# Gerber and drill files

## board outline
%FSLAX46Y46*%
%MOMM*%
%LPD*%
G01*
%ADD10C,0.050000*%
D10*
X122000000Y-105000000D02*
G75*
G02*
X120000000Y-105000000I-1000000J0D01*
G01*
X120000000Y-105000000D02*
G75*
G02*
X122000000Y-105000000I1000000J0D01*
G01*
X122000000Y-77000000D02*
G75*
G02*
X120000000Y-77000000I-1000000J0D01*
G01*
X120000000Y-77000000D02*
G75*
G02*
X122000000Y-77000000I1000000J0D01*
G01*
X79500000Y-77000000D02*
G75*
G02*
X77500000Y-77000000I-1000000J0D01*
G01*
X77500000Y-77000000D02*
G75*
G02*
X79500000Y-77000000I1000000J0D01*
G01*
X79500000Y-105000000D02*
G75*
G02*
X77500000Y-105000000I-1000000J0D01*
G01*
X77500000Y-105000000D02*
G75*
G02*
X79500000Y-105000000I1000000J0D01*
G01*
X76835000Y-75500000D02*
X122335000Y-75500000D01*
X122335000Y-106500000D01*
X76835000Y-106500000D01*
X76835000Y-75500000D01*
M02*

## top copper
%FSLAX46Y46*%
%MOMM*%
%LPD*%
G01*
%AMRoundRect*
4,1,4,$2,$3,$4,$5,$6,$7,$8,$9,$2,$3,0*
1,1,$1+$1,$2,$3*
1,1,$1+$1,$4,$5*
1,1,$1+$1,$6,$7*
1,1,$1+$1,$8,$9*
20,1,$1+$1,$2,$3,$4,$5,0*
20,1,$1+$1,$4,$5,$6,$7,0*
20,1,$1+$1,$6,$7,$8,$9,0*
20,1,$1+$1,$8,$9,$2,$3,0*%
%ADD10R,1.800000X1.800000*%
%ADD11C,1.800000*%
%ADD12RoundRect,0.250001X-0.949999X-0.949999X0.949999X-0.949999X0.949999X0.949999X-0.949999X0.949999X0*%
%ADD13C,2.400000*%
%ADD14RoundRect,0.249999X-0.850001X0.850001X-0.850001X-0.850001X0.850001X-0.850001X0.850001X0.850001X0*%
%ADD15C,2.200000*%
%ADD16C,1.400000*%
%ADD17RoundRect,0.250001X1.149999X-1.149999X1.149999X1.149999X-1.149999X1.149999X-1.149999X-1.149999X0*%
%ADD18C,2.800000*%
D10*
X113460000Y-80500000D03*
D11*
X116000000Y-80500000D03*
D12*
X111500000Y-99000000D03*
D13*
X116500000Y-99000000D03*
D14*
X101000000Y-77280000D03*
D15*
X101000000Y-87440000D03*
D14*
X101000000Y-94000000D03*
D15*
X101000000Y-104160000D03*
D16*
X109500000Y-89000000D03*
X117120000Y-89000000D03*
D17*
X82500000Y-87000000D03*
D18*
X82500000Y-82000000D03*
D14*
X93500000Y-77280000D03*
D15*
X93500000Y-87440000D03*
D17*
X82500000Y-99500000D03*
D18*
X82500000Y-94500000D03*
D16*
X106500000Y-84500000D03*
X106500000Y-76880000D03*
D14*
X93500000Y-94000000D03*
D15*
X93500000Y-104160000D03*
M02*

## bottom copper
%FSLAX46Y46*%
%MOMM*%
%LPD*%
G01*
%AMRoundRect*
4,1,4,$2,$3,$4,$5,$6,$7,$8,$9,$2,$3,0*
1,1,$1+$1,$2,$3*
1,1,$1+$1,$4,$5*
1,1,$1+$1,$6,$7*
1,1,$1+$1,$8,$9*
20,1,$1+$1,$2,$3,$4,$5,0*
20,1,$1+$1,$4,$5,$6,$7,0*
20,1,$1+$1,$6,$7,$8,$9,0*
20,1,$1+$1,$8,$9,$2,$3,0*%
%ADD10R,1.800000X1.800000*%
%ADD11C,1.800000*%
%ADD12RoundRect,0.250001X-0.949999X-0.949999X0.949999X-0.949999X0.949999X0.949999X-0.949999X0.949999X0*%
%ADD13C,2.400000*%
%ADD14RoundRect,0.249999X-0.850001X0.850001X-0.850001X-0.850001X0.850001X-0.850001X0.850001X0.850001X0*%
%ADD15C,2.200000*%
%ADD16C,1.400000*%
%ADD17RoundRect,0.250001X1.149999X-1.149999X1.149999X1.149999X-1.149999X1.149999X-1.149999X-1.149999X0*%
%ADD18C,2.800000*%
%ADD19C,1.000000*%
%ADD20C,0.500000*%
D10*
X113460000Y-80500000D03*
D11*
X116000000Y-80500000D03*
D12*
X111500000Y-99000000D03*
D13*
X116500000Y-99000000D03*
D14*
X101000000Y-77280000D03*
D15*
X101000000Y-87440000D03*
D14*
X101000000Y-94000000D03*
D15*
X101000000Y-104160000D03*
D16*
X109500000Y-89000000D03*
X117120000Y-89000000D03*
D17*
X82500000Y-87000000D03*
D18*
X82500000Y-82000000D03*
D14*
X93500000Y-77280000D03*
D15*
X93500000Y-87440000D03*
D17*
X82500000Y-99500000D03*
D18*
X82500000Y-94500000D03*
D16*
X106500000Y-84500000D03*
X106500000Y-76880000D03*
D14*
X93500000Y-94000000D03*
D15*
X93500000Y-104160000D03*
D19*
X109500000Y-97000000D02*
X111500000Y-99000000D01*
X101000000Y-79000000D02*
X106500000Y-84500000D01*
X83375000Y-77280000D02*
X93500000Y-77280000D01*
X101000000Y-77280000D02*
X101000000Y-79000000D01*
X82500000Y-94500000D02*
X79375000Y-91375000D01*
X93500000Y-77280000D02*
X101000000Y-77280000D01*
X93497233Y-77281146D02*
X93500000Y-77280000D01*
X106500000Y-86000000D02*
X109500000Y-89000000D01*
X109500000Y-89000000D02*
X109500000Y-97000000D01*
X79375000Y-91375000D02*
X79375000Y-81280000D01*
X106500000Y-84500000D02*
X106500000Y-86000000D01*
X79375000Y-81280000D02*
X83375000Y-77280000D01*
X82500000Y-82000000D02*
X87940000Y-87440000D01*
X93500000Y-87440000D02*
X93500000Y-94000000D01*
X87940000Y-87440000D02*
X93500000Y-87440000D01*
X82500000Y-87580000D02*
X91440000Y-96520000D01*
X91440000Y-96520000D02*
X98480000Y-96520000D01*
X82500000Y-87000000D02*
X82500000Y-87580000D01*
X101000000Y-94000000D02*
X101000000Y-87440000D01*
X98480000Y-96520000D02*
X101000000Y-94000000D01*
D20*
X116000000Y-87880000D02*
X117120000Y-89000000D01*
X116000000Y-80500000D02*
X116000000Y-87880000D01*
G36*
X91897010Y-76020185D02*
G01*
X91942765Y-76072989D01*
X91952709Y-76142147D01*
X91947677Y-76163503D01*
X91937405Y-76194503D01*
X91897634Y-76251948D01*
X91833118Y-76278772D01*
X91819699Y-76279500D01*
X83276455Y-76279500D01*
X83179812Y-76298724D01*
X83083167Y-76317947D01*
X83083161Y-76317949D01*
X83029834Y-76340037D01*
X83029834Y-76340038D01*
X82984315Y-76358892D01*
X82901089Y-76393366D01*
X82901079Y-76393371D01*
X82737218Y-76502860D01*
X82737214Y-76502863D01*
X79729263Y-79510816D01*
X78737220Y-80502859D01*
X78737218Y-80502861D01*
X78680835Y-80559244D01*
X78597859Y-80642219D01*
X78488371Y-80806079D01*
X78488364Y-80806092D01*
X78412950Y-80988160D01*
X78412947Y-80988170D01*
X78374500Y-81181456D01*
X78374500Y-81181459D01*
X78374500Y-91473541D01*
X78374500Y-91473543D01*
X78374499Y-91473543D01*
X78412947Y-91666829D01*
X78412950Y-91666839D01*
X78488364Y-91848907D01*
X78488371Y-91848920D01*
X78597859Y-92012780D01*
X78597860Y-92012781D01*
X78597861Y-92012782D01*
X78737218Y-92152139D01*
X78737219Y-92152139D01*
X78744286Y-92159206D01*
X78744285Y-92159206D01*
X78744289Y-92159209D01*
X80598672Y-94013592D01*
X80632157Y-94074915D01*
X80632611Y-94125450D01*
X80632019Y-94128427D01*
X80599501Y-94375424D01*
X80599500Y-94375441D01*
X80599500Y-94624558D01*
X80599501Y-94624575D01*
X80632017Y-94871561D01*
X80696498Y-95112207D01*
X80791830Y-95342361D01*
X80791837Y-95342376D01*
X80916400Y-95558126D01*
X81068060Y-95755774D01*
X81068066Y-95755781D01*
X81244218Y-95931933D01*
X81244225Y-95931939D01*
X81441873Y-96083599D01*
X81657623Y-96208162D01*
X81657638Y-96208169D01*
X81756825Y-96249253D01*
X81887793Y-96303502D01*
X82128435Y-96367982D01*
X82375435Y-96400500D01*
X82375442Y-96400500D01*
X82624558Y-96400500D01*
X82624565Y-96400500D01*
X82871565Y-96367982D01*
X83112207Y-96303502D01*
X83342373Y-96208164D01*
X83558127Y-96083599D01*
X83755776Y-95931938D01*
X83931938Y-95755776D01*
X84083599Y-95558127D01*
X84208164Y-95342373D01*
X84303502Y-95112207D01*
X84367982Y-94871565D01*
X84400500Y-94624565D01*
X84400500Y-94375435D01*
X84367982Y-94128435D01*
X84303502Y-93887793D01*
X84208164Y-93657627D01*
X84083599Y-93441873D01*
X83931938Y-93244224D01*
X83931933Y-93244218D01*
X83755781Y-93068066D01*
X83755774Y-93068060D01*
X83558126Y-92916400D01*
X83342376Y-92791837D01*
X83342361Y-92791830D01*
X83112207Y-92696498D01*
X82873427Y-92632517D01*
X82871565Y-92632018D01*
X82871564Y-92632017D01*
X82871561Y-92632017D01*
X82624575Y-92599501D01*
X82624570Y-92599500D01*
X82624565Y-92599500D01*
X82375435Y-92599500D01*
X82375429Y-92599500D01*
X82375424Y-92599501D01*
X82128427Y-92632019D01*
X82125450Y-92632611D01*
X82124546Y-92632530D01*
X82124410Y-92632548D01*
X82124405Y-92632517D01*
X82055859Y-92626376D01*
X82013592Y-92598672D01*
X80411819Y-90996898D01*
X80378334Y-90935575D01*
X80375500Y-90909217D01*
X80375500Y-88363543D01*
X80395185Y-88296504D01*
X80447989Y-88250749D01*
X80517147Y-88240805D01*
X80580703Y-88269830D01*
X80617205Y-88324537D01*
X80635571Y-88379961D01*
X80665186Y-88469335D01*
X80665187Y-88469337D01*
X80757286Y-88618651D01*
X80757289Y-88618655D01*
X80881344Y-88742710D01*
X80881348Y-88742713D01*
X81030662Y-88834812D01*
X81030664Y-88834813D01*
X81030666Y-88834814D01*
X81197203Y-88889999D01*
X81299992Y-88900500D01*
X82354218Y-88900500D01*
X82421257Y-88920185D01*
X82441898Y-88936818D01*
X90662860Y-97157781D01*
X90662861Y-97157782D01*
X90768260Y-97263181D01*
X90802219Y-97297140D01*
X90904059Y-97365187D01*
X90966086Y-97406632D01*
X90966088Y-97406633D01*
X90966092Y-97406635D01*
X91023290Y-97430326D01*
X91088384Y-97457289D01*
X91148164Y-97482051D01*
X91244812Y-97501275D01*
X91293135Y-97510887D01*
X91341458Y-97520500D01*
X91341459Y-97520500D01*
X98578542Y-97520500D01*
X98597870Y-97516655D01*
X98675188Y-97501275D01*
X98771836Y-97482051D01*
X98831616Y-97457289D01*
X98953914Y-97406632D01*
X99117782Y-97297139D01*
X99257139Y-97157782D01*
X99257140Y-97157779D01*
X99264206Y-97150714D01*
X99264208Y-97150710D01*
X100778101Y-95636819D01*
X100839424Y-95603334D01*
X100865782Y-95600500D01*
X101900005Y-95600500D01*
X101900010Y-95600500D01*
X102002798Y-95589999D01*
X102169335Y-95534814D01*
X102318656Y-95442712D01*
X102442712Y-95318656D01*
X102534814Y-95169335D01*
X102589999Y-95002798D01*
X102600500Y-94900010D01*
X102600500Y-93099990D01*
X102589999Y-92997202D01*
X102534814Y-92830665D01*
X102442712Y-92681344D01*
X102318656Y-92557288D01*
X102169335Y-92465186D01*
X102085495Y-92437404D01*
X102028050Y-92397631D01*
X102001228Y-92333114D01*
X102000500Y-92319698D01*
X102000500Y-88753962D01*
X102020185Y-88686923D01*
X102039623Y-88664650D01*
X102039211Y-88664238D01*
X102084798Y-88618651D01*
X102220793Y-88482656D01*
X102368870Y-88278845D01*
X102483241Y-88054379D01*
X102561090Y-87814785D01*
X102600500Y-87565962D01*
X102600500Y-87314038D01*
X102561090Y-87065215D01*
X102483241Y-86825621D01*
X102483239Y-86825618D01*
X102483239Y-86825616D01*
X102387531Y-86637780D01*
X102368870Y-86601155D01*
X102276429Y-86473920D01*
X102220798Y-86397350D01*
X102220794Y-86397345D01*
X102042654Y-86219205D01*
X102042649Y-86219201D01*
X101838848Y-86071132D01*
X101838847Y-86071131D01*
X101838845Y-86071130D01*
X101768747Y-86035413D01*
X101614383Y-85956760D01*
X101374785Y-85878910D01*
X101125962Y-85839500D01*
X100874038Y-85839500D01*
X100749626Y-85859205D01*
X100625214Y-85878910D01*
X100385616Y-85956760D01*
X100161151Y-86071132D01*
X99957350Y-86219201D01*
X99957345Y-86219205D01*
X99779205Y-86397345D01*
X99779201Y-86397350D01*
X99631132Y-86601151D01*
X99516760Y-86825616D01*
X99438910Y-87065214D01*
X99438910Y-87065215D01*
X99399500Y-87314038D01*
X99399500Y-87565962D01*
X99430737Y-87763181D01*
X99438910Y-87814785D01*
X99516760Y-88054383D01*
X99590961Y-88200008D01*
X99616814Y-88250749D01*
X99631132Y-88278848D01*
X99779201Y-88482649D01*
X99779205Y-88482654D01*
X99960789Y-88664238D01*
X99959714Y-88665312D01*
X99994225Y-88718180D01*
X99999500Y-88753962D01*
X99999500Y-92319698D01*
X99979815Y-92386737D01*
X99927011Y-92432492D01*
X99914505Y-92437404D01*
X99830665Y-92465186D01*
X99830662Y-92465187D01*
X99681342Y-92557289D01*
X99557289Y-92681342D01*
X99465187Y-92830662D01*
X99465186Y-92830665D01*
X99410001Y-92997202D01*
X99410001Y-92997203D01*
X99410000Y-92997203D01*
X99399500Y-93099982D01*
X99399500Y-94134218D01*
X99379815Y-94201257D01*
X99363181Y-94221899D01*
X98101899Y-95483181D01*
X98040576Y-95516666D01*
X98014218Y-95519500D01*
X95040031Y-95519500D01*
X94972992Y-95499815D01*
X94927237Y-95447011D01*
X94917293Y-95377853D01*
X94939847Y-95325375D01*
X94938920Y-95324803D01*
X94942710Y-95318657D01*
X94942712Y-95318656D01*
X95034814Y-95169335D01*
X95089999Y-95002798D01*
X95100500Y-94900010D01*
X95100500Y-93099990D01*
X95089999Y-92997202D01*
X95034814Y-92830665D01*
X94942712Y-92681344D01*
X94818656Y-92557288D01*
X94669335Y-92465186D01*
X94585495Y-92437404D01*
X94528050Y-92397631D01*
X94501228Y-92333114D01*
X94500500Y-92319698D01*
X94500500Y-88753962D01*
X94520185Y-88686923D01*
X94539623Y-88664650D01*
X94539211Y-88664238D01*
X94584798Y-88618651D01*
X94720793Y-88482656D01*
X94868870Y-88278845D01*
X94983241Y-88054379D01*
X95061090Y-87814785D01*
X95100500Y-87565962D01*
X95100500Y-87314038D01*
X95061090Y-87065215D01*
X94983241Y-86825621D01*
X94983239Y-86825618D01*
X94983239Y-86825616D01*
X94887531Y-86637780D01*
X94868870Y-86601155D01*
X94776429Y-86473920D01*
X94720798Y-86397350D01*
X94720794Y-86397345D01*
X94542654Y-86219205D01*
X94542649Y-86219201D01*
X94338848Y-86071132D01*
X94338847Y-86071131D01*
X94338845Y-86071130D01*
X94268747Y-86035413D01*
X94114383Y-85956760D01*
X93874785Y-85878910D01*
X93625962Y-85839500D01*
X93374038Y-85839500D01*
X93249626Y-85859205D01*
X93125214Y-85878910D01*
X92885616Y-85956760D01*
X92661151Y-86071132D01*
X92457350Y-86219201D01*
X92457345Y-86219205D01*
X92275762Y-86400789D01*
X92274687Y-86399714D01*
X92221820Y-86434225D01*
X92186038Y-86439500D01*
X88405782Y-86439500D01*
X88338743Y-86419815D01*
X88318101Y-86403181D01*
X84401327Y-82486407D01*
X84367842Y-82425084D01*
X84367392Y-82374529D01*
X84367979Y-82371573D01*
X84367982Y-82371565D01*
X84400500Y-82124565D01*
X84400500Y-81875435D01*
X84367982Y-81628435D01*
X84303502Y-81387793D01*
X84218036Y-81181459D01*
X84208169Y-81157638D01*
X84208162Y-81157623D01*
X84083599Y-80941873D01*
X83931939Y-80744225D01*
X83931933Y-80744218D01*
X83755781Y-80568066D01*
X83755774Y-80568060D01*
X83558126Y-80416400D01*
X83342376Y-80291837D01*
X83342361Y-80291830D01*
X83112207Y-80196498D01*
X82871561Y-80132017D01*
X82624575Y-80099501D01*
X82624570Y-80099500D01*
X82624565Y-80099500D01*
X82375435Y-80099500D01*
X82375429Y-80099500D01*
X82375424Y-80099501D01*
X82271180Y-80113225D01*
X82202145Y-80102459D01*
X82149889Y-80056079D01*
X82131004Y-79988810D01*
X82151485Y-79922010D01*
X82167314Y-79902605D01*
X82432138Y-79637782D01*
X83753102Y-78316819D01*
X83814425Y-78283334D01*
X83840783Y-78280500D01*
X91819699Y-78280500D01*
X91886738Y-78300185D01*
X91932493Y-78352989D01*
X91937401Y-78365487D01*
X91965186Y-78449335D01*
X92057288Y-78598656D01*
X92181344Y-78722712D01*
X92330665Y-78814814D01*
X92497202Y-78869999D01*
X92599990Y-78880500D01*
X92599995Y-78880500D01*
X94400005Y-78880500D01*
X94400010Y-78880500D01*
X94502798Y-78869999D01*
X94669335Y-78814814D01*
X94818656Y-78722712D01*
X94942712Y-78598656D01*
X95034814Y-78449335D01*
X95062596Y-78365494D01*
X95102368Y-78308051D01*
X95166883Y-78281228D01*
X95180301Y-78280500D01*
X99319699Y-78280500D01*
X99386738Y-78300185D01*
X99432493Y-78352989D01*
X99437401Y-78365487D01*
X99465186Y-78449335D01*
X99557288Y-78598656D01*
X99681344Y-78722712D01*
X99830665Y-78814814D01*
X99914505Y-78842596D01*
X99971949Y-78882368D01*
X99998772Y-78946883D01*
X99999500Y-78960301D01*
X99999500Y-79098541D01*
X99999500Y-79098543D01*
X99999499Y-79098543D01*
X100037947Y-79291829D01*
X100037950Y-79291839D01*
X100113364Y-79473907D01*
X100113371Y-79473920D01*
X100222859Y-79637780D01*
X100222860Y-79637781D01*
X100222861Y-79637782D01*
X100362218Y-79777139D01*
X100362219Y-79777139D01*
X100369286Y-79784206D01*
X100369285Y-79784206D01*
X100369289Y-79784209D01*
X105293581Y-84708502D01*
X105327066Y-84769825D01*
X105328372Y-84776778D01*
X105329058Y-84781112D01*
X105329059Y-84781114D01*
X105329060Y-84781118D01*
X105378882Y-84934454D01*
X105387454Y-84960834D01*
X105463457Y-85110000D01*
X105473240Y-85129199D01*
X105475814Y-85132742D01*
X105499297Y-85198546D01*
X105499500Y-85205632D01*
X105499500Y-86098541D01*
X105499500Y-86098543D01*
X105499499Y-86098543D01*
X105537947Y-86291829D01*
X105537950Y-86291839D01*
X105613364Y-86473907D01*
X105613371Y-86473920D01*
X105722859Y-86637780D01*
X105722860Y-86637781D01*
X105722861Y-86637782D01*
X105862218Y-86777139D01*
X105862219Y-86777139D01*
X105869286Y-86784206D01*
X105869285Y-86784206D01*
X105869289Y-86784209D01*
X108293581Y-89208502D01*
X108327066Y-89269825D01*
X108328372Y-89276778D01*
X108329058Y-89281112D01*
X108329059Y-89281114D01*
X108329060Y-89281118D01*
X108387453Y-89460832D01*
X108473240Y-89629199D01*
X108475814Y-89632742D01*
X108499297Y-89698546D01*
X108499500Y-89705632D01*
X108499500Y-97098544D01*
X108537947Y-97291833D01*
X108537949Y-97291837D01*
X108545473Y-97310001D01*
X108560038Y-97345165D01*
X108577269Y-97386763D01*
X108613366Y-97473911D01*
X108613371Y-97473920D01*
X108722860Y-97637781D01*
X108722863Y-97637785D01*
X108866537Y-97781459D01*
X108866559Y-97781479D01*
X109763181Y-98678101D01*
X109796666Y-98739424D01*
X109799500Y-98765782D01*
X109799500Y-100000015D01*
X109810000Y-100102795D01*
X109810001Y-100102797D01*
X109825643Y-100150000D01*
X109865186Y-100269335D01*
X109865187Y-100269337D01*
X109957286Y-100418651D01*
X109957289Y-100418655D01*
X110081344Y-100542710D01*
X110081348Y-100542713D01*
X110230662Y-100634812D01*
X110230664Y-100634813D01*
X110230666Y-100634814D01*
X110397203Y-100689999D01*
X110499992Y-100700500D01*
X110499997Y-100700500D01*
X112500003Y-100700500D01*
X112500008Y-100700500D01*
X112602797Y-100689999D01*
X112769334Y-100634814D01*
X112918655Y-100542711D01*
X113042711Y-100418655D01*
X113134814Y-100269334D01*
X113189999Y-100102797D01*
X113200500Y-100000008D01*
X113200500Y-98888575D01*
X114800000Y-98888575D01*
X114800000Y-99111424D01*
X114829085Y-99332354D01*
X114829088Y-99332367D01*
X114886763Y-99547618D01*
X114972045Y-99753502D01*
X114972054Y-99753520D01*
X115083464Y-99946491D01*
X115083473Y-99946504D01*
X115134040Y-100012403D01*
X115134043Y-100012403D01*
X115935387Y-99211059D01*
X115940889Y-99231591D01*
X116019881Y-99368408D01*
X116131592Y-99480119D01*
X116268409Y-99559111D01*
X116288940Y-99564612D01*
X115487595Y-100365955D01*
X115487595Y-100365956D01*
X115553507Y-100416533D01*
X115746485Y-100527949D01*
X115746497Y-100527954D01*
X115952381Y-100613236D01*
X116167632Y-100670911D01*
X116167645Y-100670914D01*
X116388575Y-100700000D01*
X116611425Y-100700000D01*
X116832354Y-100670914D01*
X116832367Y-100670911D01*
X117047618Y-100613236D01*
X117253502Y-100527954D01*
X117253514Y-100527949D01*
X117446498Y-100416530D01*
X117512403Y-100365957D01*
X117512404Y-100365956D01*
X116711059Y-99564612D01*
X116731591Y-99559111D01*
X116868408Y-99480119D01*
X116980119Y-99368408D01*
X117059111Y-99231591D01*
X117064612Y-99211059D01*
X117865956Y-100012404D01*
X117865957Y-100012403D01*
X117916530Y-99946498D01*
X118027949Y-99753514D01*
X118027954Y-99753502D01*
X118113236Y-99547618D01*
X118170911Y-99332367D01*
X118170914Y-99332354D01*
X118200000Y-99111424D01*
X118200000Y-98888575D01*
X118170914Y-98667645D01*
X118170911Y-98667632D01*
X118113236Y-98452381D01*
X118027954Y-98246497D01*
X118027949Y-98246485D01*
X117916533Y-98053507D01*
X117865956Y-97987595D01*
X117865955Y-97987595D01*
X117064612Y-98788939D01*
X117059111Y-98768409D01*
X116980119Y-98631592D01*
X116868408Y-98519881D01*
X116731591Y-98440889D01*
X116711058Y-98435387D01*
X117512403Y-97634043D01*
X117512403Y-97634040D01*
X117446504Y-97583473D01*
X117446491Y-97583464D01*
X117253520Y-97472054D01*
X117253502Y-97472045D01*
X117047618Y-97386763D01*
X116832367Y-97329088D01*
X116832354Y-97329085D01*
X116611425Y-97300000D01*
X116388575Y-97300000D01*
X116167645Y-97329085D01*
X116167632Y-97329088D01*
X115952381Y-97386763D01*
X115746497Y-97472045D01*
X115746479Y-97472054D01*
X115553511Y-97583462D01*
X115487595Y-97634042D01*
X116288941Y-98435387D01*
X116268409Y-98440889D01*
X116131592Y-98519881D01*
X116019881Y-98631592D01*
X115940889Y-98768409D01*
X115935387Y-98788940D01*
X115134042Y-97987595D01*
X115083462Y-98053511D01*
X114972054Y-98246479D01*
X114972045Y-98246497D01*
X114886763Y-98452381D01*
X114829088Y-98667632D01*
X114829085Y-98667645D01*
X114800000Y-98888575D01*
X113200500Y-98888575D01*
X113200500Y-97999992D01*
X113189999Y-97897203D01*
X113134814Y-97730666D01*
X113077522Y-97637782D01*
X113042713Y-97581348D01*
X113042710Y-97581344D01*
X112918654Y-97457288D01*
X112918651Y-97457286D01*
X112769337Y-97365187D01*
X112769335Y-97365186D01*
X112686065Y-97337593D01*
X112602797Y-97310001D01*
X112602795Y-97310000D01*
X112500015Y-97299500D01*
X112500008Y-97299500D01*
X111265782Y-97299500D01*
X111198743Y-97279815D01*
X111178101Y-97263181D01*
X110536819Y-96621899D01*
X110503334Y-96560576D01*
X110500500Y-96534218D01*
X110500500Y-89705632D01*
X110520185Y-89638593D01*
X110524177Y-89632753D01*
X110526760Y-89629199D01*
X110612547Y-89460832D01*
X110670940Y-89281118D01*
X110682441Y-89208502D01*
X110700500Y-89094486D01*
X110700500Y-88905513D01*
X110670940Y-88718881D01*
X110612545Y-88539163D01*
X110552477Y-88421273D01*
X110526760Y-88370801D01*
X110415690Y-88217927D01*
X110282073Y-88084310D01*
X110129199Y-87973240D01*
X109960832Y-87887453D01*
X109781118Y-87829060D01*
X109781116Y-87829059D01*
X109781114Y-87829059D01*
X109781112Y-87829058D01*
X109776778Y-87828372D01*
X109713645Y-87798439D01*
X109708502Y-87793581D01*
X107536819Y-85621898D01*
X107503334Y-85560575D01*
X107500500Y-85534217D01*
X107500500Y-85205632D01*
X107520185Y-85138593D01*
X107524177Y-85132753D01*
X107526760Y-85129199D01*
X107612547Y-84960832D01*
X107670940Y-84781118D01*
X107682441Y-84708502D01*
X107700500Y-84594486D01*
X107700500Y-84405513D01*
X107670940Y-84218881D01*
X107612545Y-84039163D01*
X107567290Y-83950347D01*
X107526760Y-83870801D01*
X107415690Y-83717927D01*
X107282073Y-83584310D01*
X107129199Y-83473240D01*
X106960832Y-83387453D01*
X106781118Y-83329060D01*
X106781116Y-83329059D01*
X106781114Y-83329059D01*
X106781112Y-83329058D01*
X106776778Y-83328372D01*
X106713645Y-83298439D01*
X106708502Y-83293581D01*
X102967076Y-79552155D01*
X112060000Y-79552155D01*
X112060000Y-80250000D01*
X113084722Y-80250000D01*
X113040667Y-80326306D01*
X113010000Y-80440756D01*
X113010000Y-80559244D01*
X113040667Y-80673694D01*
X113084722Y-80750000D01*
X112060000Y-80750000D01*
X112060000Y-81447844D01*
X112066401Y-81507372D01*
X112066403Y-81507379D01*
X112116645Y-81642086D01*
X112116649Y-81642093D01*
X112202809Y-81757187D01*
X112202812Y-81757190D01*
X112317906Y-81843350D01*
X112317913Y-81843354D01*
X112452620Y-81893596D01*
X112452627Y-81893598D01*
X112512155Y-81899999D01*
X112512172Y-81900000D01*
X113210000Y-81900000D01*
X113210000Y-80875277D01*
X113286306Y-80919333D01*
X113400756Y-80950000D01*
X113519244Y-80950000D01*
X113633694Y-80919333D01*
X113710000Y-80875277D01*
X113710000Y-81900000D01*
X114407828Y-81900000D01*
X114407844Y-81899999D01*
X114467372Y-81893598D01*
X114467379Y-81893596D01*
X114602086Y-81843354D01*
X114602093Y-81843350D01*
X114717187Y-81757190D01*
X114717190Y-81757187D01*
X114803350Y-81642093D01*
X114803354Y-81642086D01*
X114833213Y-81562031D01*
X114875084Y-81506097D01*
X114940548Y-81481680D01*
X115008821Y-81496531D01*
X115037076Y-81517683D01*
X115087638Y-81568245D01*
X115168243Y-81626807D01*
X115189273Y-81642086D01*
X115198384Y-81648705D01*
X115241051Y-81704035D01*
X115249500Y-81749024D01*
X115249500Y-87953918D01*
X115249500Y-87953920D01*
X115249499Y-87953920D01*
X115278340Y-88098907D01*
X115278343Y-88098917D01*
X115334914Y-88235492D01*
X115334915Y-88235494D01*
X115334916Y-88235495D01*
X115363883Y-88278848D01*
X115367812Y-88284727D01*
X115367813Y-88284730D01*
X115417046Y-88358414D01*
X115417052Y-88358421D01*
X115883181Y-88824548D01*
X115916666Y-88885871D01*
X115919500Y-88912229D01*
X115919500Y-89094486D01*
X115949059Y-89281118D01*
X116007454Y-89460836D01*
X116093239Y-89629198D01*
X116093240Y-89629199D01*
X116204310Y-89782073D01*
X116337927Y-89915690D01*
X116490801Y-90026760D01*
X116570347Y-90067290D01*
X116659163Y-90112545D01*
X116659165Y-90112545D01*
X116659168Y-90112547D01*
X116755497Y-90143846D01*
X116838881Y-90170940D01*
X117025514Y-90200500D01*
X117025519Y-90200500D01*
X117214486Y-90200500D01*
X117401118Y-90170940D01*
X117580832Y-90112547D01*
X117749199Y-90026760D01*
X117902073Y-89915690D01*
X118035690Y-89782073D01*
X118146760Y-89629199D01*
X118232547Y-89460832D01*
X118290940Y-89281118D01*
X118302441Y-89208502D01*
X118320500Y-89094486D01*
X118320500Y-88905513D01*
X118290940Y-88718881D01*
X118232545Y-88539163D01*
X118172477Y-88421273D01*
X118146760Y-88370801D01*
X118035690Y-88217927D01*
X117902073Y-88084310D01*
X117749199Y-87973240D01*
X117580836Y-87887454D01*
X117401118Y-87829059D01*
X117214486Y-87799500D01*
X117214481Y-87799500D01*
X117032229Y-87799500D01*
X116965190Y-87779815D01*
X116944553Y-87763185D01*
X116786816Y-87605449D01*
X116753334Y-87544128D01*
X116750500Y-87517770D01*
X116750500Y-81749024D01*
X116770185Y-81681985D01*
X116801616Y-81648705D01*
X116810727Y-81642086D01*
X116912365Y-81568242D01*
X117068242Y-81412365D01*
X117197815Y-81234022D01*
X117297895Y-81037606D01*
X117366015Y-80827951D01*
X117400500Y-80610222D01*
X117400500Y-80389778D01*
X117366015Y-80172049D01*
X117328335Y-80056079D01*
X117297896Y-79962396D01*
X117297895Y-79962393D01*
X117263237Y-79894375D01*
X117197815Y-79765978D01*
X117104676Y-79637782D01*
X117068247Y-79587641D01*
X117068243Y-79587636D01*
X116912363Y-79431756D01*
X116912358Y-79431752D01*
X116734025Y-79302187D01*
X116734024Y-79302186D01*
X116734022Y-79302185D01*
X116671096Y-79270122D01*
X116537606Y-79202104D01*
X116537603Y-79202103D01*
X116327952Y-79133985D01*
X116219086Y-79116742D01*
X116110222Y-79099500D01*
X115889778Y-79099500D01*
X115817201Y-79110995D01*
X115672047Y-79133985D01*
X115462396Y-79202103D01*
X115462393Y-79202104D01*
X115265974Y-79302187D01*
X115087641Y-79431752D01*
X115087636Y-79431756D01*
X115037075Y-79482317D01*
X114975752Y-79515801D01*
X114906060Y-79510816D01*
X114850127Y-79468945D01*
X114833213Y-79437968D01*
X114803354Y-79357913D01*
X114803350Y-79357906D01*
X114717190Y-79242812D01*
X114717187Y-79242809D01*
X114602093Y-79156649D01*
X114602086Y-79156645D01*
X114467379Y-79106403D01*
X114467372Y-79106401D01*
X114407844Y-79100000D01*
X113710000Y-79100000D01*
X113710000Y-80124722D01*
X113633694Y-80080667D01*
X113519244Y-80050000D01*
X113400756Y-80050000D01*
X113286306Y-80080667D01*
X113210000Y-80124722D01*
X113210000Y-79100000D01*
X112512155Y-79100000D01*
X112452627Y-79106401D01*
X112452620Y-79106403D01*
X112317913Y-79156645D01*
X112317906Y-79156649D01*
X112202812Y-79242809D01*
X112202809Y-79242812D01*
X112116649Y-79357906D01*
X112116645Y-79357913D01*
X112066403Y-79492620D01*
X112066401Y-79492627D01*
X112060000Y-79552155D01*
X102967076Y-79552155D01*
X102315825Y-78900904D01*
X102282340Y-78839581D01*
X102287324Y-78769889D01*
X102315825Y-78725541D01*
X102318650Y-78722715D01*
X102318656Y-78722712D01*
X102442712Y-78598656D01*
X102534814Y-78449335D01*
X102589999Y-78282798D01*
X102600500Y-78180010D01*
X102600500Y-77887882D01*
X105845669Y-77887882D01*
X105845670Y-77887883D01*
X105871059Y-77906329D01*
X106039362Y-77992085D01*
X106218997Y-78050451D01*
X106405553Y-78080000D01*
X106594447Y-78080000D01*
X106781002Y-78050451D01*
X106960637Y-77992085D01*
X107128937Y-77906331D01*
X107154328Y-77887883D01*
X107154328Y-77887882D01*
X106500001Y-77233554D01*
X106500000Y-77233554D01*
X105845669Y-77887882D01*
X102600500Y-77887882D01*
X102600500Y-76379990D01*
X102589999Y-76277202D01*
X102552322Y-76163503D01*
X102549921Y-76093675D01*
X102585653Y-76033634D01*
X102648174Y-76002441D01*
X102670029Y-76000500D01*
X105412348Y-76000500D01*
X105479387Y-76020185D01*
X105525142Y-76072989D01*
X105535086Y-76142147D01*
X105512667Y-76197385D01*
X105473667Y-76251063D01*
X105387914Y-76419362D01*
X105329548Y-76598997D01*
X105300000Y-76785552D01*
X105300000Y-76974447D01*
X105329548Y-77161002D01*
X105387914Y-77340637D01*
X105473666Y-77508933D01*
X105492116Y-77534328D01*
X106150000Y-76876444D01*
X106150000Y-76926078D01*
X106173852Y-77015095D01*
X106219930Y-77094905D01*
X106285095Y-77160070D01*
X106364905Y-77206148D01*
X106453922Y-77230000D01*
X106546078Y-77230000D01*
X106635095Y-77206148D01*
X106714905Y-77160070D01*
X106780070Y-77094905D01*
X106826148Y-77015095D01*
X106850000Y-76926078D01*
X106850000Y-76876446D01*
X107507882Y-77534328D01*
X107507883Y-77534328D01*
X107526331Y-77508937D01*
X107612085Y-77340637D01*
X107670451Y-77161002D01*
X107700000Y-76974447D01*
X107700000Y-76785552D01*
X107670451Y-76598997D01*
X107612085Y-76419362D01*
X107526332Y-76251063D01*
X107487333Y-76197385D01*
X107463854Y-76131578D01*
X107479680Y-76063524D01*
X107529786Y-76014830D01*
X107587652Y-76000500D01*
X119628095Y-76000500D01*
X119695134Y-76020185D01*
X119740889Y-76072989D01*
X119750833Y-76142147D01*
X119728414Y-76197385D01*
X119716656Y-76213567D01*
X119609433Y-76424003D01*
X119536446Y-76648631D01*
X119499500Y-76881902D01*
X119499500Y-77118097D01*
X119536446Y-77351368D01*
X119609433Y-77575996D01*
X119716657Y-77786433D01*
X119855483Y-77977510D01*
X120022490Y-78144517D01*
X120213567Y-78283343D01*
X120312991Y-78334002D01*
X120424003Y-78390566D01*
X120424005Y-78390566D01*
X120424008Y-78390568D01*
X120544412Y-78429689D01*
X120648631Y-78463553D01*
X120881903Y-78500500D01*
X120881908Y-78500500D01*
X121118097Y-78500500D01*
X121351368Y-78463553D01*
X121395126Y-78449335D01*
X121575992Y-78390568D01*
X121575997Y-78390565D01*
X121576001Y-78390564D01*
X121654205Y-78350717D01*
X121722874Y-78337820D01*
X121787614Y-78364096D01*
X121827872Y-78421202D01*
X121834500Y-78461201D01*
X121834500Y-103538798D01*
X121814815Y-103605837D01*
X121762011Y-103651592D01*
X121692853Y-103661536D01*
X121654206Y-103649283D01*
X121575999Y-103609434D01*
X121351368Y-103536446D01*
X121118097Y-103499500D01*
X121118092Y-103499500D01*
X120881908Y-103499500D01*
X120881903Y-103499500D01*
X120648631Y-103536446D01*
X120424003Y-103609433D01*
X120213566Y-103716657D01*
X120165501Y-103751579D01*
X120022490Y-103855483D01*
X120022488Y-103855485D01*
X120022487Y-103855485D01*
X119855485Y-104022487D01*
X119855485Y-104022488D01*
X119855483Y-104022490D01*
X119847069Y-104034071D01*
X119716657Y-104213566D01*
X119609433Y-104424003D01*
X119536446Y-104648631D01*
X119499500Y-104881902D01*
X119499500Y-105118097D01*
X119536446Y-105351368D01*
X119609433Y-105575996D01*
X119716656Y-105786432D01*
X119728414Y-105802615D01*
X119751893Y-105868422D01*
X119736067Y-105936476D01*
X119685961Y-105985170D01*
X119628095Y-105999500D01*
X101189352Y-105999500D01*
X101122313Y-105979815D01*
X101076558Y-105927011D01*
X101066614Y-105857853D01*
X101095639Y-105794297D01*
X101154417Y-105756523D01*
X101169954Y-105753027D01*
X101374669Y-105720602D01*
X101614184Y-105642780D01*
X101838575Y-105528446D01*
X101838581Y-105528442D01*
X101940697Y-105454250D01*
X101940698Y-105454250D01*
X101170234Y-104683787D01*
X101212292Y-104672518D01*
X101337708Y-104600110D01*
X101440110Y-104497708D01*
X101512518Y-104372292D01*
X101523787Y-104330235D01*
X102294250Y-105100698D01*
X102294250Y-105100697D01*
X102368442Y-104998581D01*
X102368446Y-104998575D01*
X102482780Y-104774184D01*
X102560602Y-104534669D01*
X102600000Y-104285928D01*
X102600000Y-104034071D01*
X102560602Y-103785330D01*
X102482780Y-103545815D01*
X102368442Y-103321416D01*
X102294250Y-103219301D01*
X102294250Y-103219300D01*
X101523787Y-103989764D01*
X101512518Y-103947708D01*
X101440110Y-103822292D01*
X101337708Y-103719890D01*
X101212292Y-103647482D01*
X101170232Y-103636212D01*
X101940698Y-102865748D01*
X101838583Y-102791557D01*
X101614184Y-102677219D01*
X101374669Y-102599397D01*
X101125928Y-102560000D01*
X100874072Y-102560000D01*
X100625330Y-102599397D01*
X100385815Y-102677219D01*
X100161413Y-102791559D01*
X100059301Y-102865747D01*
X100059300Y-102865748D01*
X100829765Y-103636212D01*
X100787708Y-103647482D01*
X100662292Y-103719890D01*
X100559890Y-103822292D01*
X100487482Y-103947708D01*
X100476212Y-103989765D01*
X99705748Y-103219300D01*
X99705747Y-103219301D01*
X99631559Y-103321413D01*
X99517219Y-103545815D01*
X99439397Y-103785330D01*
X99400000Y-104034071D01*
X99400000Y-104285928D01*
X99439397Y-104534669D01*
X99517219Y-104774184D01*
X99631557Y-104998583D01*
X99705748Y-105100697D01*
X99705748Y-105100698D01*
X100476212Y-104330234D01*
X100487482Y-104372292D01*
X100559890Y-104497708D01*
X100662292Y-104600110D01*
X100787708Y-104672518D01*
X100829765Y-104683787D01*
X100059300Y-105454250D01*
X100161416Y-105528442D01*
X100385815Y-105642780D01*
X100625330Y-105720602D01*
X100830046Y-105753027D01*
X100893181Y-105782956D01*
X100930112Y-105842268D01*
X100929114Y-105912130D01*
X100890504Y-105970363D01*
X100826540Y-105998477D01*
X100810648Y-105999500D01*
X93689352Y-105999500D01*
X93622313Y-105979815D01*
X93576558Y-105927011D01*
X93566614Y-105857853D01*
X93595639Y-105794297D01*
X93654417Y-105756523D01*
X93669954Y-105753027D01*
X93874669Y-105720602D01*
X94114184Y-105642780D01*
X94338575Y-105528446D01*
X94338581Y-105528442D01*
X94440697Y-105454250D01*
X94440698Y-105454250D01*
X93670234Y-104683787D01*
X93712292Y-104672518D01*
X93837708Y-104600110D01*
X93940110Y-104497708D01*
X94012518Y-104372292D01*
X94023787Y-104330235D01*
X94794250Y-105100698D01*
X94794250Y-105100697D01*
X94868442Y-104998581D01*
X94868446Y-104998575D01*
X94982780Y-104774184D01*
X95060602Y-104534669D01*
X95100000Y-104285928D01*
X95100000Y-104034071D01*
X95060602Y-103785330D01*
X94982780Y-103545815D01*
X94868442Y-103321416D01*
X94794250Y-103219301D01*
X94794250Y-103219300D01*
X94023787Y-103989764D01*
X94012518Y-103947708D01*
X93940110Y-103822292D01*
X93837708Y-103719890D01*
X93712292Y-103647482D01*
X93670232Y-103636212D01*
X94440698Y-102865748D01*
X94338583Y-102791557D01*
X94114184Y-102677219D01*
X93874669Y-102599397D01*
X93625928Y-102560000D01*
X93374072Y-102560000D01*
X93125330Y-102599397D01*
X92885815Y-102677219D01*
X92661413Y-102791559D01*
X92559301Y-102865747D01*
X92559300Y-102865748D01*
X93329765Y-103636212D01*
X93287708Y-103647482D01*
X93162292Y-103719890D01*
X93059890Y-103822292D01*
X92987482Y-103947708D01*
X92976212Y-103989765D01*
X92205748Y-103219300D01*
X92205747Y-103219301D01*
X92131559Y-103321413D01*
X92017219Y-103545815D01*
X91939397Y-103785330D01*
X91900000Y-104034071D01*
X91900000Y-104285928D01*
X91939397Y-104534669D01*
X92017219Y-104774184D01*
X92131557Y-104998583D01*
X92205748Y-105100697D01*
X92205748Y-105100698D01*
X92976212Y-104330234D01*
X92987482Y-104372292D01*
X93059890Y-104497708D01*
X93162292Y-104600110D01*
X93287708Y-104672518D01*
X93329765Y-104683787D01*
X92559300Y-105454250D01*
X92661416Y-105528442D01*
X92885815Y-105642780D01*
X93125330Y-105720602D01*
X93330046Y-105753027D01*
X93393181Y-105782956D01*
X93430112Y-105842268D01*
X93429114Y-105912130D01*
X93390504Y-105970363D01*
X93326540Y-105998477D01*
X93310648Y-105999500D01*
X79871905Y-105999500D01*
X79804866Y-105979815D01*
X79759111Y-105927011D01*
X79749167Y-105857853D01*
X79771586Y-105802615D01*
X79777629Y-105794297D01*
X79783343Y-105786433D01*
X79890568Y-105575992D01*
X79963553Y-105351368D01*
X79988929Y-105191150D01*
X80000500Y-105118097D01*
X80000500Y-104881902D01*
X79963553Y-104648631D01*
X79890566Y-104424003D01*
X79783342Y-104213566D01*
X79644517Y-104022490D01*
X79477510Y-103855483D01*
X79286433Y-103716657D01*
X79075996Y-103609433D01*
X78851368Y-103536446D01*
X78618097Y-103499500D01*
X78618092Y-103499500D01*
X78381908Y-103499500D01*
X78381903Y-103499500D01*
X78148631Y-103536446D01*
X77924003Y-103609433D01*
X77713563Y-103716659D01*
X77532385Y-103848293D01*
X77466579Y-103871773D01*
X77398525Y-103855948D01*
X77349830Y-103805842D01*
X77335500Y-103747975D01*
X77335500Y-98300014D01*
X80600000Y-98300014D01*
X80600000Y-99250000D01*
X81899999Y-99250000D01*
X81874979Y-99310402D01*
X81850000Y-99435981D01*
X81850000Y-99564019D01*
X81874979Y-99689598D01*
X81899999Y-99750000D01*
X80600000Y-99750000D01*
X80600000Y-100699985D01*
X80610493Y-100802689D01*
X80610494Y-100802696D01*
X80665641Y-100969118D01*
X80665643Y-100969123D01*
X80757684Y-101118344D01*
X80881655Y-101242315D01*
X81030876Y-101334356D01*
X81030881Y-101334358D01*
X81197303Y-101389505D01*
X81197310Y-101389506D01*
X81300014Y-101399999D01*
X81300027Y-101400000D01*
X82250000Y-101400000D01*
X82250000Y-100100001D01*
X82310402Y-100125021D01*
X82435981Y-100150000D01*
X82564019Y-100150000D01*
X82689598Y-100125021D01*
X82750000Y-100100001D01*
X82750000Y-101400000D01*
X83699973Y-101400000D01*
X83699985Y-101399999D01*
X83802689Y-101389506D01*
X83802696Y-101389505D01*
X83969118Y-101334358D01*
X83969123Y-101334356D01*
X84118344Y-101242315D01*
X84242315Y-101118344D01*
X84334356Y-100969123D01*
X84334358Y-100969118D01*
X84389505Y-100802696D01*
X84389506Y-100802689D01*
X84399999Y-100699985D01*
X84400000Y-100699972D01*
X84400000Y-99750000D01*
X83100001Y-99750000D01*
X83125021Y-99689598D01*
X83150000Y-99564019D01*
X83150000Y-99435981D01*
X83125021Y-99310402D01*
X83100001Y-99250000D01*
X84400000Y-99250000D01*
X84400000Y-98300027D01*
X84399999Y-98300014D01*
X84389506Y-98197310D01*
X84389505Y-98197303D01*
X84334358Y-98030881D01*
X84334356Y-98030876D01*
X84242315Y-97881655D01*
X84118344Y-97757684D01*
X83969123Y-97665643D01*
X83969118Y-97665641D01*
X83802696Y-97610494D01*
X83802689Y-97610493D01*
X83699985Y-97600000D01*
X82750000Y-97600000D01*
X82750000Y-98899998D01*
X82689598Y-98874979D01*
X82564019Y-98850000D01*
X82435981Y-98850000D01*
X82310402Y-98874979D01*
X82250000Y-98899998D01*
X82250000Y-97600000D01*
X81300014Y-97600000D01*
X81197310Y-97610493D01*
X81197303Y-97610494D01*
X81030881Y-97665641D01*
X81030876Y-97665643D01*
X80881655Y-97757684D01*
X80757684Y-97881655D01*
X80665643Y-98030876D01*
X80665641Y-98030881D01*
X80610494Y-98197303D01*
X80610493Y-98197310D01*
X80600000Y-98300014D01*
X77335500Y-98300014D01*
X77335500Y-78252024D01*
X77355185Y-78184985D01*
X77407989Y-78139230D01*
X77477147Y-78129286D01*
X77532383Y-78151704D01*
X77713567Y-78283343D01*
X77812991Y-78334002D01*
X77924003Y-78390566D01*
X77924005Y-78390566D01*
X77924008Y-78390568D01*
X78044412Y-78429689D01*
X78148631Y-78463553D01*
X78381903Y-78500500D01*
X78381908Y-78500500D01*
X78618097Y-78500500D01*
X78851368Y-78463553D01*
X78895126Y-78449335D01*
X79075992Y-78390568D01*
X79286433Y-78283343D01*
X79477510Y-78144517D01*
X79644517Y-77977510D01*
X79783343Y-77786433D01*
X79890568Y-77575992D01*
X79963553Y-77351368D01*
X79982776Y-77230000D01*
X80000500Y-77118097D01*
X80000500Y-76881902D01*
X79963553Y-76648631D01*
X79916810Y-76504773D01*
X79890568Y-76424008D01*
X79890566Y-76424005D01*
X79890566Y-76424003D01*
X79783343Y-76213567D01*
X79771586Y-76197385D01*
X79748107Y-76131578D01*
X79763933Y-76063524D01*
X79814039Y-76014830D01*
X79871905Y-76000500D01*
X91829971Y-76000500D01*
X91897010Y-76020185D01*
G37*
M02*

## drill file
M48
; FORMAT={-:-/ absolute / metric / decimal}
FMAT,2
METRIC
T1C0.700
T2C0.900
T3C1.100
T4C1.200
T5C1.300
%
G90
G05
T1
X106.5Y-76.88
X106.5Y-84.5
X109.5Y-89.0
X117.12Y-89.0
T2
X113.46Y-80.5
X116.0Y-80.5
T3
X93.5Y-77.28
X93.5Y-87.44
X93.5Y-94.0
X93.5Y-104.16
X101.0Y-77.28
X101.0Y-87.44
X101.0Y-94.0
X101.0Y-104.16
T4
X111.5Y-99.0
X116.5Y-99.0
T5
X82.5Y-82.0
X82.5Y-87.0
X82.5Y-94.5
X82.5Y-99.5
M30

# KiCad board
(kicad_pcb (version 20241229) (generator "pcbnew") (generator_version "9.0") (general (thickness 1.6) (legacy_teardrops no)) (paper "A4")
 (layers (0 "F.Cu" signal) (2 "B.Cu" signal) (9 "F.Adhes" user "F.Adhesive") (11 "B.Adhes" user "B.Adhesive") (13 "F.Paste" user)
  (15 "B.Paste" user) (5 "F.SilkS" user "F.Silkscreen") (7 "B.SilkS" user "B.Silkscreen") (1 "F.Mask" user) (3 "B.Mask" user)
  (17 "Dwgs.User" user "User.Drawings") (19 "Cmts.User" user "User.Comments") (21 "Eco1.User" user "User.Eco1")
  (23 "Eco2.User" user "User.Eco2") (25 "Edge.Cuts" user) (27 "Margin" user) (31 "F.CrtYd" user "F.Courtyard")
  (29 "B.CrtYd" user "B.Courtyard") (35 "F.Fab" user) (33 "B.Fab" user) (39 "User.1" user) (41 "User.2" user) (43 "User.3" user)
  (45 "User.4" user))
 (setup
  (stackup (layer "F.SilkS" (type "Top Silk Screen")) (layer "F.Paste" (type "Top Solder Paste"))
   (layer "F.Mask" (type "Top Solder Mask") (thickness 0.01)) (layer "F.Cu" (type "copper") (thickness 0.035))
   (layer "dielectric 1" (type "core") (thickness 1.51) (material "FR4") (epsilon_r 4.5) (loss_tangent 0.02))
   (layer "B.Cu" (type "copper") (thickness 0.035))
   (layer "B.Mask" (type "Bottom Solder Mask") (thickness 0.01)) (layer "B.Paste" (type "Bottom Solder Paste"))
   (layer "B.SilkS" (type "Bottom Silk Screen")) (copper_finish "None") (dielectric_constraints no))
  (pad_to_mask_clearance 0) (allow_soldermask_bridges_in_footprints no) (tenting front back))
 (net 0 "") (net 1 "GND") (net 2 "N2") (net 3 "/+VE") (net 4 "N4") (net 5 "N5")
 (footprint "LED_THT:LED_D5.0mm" (layer "F.Cu") (at 113.46 80.5)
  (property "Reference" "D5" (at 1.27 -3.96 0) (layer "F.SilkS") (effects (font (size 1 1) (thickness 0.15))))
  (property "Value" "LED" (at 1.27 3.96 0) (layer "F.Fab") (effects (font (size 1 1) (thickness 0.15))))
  (pad "1" thru_hole rect (at 0 0) (size 1.8 1.8) (drill 0.9) (layers "*.Cu" "*.Mask") (remove_unused_layers no) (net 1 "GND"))
  (pad "2" thru_hole circle (at 2.54 0) (size 1.8 1.8) (drill 0.9) (layers "*.Cu" "*.Mask") (remove_unused_layers no) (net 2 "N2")))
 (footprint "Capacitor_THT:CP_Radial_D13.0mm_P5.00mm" (layer "F.Cu") (at 111.5 99)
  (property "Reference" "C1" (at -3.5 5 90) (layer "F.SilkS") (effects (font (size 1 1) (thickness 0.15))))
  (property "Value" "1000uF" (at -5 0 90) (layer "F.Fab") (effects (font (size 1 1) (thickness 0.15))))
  (pad "1" thru_hole roundrect (at 0 0) (size 2.4 2.4) (drill 1.2) (layers "*.Cu" "*.Mask") (remove_unused_layers no)
   (roundrect_rratio 0.104167) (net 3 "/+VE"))
  (pad "2" thru_hole circle (at 5 0) (size 2.4 2.4) (drill 1.2) (layers "*.Cu" "*.Mask") (remove_unused_layers no) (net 1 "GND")))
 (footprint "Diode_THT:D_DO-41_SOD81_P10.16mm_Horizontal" (layer "F.Cu") (at 101 77.28 -90)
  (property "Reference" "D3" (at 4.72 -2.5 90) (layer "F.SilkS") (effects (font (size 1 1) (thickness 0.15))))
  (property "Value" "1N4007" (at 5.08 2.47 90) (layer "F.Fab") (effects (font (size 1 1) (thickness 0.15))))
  (pad "1" thru_hole roundrect (at 0 0 270) (size 2.2 2.2) (drill 1.1) (layers "*.Cu" "*.Mask") (remove_unused_layers no)
   (roundrect_rratio 0.113636) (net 3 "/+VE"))
  (pad "2" thru_hole circle (at 10.16 0 270) (size 2.2 2.2) (drill 1.1) (layers "*.Cu" "*.Mask") (remove_unused_layers no) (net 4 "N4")))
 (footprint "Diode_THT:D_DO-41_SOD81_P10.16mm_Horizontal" (layer "F.Cu") (at 101 94 -90)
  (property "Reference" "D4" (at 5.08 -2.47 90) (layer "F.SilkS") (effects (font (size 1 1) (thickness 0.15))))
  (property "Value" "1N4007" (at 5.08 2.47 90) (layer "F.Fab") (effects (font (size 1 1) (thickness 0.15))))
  (pad "1" thru_hole roundrect (at 0 0 270) (size 2.2 2.2) (drill 1.1) (layers "*.Cu" "*.Mask") (remove_unused_layers no)
   (roundrect_rratio 0.113636) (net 4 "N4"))
  (pad "2" thru_hole circle (at 10.16 0 270) (size 2.2 2.2) (drill 1.1) (layers "*.Cu" "*.Mask") (remove_unused_layers no) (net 1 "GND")))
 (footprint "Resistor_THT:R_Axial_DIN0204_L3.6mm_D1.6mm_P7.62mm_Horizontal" (layer "F.Cu") (at 109.5 89)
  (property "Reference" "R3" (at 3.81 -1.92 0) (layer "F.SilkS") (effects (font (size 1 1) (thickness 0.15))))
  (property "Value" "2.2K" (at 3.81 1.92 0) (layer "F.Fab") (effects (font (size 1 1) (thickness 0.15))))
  (pad "1" thru_hole circle (at 0 0) (size 1.4 1.4) (drill 0.7) (layers "*.Cu" "*.Mask") (remove_unused_layers no) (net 3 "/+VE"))
  (pad "2" thru_hole circle (at 7.62 0) (size 1.4 1.4) (drill 0.7) (layers "*.Cu" "*.Mask") (remove_unused_layers no) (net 2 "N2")))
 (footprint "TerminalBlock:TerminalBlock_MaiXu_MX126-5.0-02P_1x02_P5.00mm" (layer "F.Cu") (at 82.5 87 90)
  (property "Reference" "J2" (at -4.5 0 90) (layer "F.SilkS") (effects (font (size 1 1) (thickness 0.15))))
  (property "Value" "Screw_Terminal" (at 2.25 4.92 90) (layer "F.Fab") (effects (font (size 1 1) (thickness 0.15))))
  (pad "1" thru_hole roundrect (at 0 0 90) (size 2.8 2.8) (drill 1.3) (layers "*.Cu" "*.Mask") (remove_unused_layers no)
   (roundrect_rratio 0.089286) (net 4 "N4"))
  (pad "2" thru_hole circle (at 5 0 90) (size 2.8 2.8) (drill 1.3) (layers "*.Cu" "*.Mask") (remove_unused_layers no) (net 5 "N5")))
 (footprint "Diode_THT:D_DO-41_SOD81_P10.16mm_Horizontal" (layer "F.Cu") (at 93.5 77.28 -90)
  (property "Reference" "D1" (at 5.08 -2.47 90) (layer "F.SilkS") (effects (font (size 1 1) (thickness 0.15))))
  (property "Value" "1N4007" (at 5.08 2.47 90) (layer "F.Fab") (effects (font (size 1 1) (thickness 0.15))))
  (pad "1" thru_hole roundrect (at 0 0 270) (size 2.2 2.2) (drill 1.1) (layers "*.Cu" "*.Mask") (remove_unused_layers no)
   (roundrect_rratio 0.113636) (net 3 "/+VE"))
  (pad "2" thru_hole circle (at 10.16 0 270) (size 2.2 2.2) (drill 1.1) (layers "*.Cu" "*.Mask") (remove_unused_layers no) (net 5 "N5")))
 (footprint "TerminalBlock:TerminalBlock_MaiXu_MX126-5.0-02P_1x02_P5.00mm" (layer "F.Cu") (at 82.5 99.5 90)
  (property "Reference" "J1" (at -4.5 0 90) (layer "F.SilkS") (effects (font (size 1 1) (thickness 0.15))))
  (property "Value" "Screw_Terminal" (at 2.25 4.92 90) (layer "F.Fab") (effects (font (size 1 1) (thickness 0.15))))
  (pad "1" thru_hole roundrect (at 0 0 90) (size 2.8 2.8) (drill 1.3) (layers "*.Cu" "*.Mask") (remove_unused_layers no)
   (roundrect_rratio 0.089286) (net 1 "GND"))
  (pad "2" thru_hole circle (at 5 0 90) (size 2.8 2.8) (drill 1.3) (layers "*.Cu" "*.Mask") (remove_unused_layers no) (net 3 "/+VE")))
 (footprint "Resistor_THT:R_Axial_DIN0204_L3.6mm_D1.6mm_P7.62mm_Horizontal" (layer "F.Cu") (at 106.5 84.5 90)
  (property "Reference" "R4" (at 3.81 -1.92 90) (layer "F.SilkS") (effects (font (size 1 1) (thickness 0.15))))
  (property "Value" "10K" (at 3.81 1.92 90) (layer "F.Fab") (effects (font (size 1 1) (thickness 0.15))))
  (pad "1" thru_hole circle (at 0 0 90) (size 1.4 1.4) (drill 0.7) (layers "*.Cu" "*.Mask") (remove_unused_layers no) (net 3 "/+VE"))
  (pad "2" thru_hole circle (at 7.62 0 90) (size 1.4 1.4) (drill 0.7) (layers "*.Cu" "*.Mask") (remove_unused_layers no) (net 1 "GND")))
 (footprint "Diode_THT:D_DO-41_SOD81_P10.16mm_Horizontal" (layer "F.Cu") (at 93.5 94 -90)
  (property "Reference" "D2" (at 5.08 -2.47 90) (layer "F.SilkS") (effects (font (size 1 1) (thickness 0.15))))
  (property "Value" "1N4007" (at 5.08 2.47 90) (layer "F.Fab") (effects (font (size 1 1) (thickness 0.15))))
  (pad "1" thru_hole roundrect (at 0 0 270) (size 2.2 2.2) (drill 1.1) (layers "*.Cu" "*.Mask") (remove_unused_layers no)
   (roundrect_rratio 0.113636) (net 5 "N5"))
  (pad "2" thru_hole circle (at 10.16 0 270) (size 2.2 2.2) (drill 1.1) (layers "*.Cu" "*.Mask") (remove_unused_layers no) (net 1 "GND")))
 (gr_circle (center 121 105) (end 121 106) (stroke (width 0.05) (type default)) (fill no) (layer "Edge.Cuts"))
 (gr_circle (center 121 77) (end 121 78) (stroke (width 0.05) (type default)) (fill no) (layer "Edge.Cuts"))
 (gr_circle (center 78.5 77) (end 77.5 77) (stroke (width 0.05) (type default)) (fill no) (layer "Edge.Cuts"))
 (gr_circle (center 78.5 105) (end 79.5 105) (stroke (width 0.05) (type default)) (fill no) (layer "Edge.Cuts"))
 (gr_rect (start 76.835 75.5) (end 122.335 106.5) (stroke (width 0.05) (type default)) (fill no) (layer "Edge.Cuts"))
 (segment (start 109.5 97) (end 111.5 99) (width 1) (layer "B.Cu") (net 3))
 (segment (start 101 79) (end 106.5 84.5) (width 1) (layer "B.Cu") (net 3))
 (segment (start 83.375 77.28) (end 93.5 77.28) (width 1) (layer "B.Cu") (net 3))
 (segment (start 101 77.28) (end 101 79) (width 1) (layer "B.Cu") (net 3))
 (segment (start 82.5 94.5) (end 79.375 91.375) (width 1) (layer "B.Cu") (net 3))
 (segment (start 93.5 77.28) (end 101 77.28) (width 1) (layer "B.Cu") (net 3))
 (segment (start 93.497233 77.281146) (end 93.5 77.28) (width 1) (layer "B.Cu") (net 3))
 (segment (start 106.5 86) (end 109.5 89) (width 1) (layer "B.Cu") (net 3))
 (segment (start 109.5 89) (end 109.5 97) (width 1) (layer "B.Cu") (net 3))
 (segment (start 79.375 91.375) (end 79.375 81.28) (width 1) (layer "B.Cu") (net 3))
 (segment (start 106.5 84.5) (end 106.5 86) (width 1) (layer "B.Cu") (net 3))
 (segment (start 79.375 81.28) (end 83.375 77.28) (width 1) (layer "B.Cu") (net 3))
 (segment (start 82.5 82) (end 87.94 87.44) (width 1) (layer "B.Cu") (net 5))
 (segment (start 93.5 87.44) (end 93.5 94) (width 1) (layer "B.Cu") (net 5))
 (segment (start 87.94 87.44) (end 93.5 87.44) (width 1) (layer "B.Cu") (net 5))
 (segment (start 82.5 87.58) (end 91.44 96.52) (width 1) (layer "B.Cu") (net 4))
 (segment (start 91.44 96.52) (end 98.48 96.52) (width 1) (layer "B.Cu") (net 4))
 (segment (start 82.5 87) (end 82.5 87.58) (width 1) (layer "B.Cu") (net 4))
 (segment (start 101 94) (end 101 87.44) (width 1) (layer "B.Cu") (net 4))
 (segment (start 98.48 96.52) (end 101 94) (width 1) (layer "B.Cu") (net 4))
 (segment (start 116 87.88) (end 117.12 89) (width 0.5) (layer "B.Cu") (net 2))
 (segment (start 116 80.5) (end 116 87.88) (width 0.5) (layer "B.Cu") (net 2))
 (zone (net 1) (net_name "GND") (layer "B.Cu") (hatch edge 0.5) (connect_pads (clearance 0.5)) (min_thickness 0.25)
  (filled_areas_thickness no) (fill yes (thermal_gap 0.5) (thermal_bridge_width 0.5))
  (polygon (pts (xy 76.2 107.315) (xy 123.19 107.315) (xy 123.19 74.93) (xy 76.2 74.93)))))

